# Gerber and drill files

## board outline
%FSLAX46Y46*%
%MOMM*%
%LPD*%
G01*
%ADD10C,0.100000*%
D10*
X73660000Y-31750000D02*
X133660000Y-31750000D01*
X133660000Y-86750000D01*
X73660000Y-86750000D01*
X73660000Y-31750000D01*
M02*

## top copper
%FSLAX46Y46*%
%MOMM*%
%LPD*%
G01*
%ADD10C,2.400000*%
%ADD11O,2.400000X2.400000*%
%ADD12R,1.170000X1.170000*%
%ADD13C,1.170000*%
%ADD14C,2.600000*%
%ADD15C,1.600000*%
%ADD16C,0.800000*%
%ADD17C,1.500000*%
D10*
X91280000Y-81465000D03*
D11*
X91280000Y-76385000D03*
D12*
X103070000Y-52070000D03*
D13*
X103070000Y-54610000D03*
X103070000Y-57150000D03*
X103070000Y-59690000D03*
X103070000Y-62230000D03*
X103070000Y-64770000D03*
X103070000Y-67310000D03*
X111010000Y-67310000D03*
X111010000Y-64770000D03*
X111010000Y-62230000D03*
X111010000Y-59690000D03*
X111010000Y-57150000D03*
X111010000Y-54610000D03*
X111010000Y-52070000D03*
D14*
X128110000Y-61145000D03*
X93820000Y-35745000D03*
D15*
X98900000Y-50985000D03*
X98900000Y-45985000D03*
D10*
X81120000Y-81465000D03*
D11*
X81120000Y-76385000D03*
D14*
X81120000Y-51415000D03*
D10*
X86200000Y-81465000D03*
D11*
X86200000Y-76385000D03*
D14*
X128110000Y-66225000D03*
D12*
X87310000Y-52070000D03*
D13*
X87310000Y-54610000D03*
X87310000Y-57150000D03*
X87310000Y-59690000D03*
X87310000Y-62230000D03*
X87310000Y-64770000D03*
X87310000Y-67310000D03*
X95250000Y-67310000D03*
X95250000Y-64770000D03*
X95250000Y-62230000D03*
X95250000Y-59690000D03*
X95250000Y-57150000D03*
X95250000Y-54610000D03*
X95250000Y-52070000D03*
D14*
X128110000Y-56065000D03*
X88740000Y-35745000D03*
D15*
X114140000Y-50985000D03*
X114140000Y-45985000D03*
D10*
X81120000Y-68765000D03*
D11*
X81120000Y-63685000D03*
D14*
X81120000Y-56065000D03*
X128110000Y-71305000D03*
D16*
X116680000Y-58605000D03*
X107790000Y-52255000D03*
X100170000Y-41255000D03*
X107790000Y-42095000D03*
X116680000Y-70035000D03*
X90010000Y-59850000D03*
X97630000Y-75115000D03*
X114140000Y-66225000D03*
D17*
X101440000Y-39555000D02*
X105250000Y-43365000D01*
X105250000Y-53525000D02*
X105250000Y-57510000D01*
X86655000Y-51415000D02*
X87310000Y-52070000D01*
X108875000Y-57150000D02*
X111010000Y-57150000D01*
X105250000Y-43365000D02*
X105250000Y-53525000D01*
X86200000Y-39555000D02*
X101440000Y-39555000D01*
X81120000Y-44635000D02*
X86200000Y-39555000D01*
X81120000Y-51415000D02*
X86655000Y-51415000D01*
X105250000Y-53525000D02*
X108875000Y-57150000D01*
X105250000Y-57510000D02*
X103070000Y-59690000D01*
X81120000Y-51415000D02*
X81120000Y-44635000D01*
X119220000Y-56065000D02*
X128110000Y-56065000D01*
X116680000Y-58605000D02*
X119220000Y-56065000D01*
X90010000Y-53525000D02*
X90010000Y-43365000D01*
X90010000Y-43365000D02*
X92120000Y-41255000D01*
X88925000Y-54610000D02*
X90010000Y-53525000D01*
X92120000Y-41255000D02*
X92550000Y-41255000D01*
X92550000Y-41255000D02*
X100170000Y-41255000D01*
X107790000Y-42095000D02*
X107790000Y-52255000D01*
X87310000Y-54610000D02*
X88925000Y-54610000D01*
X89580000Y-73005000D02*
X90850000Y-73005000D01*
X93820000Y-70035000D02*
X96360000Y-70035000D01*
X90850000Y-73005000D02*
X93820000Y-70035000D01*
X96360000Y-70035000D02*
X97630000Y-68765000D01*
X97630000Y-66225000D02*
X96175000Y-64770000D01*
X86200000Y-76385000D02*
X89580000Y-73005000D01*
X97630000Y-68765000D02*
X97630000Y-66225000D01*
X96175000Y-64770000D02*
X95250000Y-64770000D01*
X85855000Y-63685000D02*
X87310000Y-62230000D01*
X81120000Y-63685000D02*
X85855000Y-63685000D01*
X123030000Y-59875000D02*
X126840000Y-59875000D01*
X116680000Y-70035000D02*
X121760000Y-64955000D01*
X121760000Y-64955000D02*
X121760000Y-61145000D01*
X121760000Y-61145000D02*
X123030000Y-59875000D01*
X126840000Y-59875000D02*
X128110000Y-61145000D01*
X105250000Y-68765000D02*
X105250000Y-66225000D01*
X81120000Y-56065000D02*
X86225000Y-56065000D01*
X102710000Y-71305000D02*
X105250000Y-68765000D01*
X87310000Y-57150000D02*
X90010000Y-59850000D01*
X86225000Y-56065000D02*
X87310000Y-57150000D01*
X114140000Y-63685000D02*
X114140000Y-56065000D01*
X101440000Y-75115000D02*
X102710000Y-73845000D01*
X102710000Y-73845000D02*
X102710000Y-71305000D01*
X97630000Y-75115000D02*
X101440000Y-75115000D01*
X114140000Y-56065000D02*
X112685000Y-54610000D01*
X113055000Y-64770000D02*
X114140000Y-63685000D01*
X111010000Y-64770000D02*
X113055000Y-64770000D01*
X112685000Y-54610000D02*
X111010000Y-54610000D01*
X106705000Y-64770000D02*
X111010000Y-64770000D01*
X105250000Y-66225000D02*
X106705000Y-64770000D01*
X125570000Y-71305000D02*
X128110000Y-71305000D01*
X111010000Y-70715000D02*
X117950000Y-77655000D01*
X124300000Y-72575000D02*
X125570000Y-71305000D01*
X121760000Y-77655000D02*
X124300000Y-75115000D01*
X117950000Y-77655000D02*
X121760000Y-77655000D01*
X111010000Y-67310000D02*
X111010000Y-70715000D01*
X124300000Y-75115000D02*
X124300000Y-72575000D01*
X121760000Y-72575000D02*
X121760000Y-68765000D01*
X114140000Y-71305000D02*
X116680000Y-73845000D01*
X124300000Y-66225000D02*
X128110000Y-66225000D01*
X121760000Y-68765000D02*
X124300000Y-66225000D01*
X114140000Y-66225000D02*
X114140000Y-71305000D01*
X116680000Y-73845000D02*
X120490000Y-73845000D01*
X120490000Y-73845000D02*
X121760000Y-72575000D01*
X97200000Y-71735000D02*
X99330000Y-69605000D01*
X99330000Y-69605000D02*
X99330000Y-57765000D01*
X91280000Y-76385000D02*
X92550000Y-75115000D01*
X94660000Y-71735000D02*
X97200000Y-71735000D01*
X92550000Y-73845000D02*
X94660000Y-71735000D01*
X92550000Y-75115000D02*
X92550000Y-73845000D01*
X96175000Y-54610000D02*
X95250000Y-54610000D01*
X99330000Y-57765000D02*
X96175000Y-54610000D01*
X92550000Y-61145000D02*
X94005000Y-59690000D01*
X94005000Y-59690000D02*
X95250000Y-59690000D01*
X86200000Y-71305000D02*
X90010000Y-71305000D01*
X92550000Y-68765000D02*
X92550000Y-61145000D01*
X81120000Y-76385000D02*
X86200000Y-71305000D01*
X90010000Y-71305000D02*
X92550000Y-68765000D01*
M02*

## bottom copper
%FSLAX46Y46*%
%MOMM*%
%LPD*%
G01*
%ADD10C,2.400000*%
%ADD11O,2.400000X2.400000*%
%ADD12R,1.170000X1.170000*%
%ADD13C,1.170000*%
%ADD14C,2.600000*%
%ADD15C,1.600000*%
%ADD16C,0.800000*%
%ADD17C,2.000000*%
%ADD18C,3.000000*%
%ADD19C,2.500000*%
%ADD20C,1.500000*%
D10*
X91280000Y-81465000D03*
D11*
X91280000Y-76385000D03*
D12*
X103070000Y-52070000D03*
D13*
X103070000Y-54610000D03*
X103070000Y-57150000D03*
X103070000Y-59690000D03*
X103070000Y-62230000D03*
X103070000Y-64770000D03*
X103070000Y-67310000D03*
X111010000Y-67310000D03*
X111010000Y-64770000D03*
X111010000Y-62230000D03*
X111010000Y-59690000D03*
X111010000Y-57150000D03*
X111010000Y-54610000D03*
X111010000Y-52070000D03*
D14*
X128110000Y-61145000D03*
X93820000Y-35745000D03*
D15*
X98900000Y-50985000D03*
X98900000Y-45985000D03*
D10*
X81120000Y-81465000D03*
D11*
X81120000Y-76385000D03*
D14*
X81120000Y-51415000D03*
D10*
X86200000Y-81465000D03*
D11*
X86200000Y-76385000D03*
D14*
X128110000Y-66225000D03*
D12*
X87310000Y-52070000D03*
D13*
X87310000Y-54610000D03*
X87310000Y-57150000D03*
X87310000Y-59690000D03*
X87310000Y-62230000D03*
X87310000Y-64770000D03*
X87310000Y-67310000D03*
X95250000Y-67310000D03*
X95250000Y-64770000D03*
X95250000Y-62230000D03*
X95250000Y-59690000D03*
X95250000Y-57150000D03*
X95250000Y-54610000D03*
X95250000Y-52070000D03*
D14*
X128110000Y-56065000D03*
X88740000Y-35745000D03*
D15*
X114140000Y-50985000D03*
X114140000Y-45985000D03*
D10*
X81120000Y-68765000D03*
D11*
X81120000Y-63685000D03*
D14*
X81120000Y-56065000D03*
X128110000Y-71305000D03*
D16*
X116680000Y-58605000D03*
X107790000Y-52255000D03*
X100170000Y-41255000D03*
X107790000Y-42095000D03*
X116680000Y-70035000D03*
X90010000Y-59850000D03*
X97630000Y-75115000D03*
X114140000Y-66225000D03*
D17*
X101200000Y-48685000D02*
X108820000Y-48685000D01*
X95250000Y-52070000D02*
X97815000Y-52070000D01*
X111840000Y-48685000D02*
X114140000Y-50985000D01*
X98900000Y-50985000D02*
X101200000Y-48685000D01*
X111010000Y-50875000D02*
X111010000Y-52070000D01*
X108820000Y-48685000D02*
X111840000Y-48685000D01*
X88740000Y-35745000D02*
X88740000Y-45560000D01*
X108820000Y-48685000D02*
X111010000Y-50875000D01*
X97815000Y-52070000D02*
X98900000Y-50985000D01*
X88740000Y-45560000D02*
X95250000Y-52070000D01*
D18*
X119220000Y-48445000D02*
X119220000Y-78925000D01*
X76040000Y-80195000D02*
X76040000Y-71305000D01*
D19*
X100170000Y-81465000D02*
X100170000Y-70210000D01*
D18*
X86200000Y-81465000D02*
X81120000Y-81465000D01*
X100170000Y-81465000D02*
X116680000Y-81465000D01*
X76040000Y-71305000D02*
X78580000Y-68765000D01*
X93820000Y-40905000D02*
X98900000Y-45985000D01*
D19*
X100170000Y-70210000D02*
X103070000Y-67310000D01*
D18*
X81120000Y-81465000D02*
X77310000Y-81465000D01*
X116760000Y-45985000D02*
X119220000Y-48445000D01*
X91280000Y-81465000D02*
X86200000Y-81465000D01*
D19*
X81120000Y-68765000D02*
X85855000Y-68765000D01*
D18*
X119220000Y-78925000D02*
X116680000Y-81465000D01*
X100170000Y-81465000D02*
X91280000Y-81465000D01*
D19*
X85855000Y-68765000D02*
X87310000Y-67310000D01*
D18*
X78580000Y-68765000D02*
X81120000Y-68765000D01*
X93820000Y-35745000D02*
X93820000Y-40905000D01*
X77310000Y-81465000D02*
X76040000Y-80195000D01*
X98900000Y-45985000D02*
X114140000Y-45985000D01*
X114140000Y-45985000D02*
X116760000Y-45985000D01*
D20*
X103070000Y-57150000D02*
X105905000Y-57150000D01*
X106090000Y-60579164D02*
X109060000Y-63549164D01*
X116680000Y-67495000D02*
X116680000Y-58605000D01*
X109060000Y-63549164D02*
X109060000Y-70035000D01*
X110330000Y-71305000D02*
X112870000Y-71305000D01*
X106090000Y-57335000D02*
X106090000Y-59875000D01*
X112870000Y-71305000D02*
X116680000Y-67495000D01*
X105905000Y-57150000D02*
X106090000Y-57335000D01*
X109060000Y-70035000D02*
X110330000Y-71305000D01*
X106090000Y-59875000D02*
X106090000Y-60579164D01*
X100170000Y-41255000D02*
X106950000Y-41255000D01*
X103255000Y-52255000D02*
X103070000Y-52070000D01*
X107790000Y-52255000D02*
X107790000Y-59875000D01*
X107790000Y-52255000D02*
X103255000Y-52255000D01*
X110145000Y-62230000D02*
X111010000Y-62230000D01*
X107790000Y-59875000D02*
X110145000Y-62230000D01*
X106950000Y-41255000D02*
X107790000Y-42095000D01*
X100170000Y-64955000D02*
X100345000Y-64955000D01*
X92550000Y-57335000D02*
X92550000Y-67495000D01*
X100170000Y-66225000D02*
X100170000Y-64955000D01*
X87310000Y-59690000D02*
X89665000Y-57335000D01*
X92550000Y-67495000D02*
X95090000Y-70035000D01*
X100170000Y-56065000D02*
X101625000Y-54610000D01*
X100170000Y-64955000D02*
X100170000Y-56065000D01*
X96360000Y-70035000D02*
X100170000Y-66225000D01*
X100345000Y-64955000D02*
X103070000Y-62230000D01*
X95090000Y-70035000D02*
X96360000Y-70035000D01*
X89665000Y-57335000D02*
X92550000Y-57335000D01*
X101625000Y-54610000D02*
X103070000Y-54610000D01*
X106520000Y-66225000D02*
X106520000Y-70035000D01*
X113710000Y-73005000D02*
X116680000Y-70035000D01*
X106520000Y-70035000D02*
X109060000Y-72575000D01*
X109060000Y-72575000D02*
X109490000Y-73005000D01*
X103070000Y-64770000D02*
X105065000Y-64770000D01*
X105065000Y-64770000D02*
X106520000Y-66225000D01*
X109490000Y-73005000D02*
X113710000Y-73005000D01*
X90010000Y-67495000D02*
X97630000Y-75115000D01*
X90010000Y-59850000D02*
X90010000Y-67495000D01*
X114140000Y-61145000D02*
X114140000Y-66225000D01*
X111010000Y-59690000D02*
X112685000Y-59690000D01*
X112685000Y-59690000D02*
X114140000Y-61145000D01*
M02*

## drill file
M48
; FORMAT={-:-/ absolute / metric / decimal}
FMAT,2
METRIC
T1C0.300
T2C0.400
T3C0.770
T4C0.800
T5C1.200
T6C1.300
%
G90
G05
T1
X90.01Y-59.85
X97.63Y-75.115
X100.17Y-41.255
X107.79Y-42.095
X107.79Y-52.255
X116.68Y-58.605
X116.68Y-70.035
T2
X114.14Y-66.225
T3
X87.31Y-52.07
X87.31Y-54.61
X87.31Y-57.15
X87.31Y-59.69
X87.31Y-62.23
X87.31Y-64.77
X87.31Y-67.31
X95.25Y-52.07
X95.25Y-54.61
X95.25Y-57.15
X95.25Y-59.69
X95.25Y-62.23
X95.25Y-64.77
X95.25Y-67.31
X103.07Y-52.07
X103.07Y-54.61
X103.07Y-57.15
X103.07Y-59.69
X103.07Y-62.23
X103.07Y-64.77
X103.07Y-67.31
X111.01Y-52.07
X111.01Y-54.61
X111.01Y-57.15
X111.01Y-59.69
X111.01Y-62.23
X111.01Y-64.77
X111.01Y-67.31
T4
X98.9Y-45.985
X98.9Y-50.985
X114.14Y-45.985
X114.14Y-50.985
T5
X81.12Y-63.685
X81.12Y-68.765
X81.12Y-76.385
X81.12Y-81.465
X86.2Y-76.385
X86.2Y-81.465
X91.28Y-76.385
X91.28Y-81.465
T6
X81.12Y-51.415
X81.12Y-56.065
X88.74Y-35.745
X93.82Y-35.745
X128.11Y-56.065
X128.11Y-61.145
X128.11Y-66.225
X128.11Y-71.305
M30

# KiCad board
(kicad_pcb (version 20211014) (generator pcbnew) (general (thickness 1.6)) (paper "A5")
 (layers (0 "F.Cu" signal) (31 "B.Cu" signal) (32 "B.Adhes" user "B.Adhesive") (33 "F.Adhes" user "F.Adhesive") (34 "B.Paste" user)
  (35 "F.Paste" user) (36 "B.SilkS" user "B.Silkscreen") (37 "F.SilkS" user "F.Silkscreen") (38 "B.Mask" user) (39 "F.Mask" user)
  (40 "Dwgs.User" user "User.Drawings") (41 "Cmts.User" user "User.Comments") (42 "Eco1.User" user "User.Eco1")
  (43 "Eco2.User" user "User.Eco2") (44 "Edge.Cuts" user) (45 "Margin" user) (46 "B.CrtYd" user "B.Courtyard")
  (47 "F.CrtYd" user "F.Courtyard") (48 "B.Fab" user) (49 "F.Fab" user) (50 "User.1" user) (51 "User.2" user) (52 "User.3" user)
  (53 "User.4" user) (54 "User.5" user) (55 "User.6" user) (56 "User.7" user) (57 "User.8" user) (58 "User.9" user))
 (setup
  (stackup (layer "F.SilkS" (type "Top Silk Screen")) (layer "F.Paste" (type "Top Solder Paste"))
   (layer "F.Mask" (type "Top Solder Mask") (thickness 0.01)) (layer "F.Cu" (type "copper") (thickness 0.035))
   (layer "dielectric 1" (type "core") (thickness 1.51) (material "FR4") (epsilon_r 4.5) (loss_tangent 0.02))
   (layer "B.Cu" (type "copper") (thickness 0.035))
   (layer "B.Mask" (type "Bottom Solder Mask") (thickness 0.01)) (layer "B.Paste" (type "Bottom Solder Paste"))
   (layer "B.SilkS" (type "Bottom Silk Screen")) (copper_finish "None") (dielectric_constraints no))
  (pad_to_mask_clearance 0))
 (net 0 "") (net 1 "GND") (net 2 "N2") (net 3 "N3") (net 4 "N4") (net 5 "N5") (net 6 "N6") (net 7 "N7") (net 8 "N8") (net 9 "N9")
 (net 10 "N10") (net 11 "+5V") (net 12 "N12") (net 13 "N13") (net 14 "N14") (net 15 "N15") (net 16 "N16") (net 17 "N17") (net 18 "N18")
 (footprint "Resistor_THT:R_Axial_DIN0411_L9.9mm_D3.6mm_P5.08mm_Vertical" (layer "F.Cu") (at 91.28 81.465 90)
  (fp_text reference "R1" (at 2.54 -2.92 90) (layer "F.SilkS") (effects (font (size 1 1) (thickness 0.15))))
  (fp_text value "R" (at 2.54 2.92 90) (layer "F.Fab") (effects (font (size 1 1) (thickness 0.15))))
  (pad "1" thru_hole circle (at 0 0 90) (size 2.4 2.4) (drill 1.2) (layers *.Cu *.Mask) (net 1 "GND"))
  (pad "2" thru_hole oval (at 5.08 0 90) (size 2.4 2.4) (drill 1.2) (layers *.Cu *.Mask) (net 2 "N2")))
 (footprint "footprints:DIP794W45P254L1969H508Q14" (layer "F.Cu") (at 107.04 59.69)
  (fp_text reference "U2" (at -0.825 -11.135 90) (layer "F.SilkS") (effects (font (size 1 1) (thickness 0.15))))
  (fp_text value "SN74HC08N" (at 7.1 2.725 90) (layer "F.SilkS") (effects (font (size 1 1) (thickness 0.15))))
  (pad "1" thru_hole rect locked (at -3.97 -7.62) (size 1.17 1.17) (drill 0.77) (layers *.Cu *.Mask) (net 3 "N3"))
  (pad "2" thru_hole circle locked (at -3.97 -5.08) (size 1.17 1.17) (drill 0.77) (layers *.Cu *.Mask) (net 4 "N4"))
  (pad "3" thru_hole circle locked (at -3.97 -2.54) (size 1.17 1.17) (drill 0.77) (layers *.Cu *.Mask) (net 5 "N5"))
  (pad "4" thru_hole circle locked (at -3.97 0) (size 1.17 1.17) (drill 0.77) (layers *.Cu *.Mask) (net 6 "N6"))
  (pad "5" thru_hole circle locked (at -3.97 2.54) (size 1.17 1.17) (drill 0.77) (layers *.Cu *.Mask) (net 4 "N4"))
  (pad "6" thru_hole circle locked (at -3.97 5.08) (size 1.17 1.17) (drill 0.77) (layers *.Cu *.Mask) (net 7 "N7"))
  (pad "7" thru_hole circle locked (at -3.97 7.62) (size 1.17 1.17) (drill 0.77) (layers *.Cu *.Mask) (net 1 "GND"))
  (pad "8" thru_hole circle locked (at 3.97 7.62) (size 1.17 1.17) (drill 0.77) (layers *.Cu *.Mask) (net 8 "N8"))
  (pad "9" thru_hole circle locked (at 3.97 5.08) (size 1.17 1.17) (drill 0.77) (layers *.Cu *.Mask) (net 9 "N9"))
  (pad "10" thru_hole circle locked (at 3.97 2.54) (size 1.17 1.17) (drill 0.77) (layers *.Cu *.Mask) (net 3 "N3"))
  (pad "11" thru_hole circle locked (at 3.97 0) (size 1.17 1.17) (drill 0.77) (layers *.Cu *.Mask) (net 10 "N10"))
  (pad "12" thru_hole circle locked (at 3.97 -2.54) (size 1.17 1.17) (drill 0.77) (layers *.Cu *.Mask) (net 6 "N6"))
  (pad "13" thru_hole circle locked (at 3.97 -5.08) (size 1.17 1.17) (drill 0.77) (layers *.Cu *.Mask) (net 9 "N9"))
  (pad "14" thru_hole circle locked (at 3.97 -7.62) (size 1.17 1.17) (drill 0.77) (layers *.Cu *.Mask) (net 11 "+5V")))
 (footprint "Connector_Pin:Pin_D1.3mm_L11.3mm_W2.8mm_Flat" (layer "F.Cu") (at 128.11 61.145)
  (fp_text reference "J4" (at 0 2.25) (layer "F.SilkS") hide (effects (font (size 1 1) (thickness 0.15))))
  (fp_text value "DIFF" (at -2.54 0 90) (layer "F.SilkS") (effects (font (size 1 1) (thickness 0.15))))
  (pad "1" thru_hole circle (at 0 0) (size 2.6 2.6) (drill 1.3) (layers *.Cu *.Mask) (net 7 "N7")))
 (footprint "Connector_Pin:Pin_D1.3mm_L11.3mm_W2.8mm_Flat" (layer "F.Cu") (at 93.82 35.745)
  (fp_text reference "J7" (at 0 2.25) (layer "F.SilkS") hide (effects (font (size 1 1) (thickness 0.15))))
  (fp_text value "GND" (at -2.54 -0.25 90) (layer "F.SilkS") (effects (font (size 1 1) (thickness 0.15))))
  (pad "1" thru_hole circle (at 0 0) (size 2.6 2.6) (drill 1.3) (layers *.Cu *.Mask) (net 1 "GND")))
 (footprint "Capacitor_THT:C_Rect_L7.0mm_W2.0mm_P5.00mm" (layer "F.Cu") (at 98.9 50.985 90)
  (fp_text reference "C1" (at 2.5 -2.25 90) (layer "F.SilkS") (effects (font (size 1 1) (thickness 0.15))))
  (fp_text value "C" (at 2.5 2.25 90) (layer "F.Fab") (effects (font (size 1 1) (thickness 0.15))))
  (pad "1" thru_hole circle (at 0 0 90) (size 1.6 1.6) (drill 0.8) (layers *.Cu *.Mask) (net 11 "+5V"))
  (pad "2" thru_hole circle (at 5 0 90) (size 1.6 1.6) (drill 0.8) (layers *.Cu *.Mask) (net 1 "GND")))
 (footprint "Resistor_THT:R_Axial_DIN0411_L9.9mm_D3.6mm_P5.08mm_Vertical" (layer "F.Cu") (at 81.12 81.465 90)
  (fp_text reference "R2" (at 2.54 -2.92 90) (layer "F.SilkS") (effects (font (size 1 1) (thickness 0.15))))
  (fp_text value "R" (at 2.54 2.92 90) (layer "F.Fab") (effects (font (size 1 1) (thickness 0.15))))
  (pad "1" thru_hole circle (at 0 0 90) (size 2.4 2.4) (drill 1.2) (layers *.Cu *.Mask) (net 1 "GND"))
  (pad "2" thru_hole oval (at 5.08 0 90) (size 2.4 2.4) (drill 1.2) (layers *.Cu *.Mask) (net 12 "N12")))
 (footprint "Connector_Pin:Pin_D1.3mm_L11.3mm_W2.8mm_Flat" (layer "F.Cu") (at 81.12 51.415 180)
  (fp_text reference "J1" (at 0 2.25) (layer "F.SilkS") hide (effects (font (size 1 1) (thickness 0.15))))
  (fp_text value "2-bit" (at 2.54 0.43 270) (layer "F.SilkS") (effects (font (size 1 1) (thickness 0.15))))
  (pad "1" thru_hole circle (at 0 0 180) (size 2.6 2.6) (drill 1.3) (layers *.Cu *.Mask) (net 6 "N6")))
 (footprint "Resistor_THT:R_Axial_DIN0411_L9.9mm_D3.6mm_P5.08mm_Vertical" (layer "F.Cu") (at 86.2 81.465 90)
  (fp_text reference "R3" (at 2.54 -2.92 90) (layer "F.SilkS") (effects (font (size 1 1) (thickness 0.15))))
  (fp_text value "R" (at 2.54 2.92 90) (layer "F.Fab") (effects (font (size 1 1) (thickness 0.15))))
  (pad "1" thru_hole circle (at 0 0 90) (size 2.4 2.4) (drill 1.2) (layers *.Cu *.Mask) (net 1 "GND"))
  (pad "2" thru_hole oval (at 5.08 0 90) (size 2.4 2.4) (drill 1.2) (layers *.Cu *.Mask) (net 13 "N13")))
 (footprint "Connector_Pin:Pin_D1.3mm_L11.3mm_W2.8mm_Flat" (layer "F.Cu") (at 128.11 66.225)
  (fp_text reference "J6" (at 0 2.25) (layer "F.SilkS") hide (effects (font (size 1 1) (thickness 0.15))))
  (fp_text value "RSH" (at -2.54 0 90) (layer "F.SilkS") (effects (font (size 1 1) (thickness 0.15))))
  (pad "1" thru_hole circle (at 0 0) (size 2.6 2.6) (drill 1.3) (layers *.Cu *.Mask) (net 10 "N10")))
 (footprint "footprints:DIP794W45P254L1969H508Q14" (layer "F.Cu") (at 91.28 59.69)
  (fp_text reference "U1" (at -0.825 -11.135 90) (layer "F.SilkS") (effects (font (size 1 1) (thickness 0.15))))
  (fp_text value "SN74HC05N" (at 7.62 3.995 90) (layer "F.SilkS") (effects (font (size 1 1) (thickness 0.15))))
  (pad "1" thru_hole rect locked (at -3.97 -7.62) (size 1.17 1.17) (drill 0.77) (layers *.Cu *.Mask) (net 6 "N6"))
  (pad "2" thru_hole circle locked (at -3.97 -5.08) (size 1.17 1.17) (drill 0.77) (layers *.Cu *.Mask) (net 3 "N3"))
  (pad "3" thru_hole circle locked (at -3.97 -2.54) (size 1.17 1.17) (drill 0.77) (layers *.Cu *.Mask) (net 9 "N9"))
  (pad "4" thru_hole circle locked (at -3.97 0) (size 1.17 1.17) (drill 0.77) (layers *.Cu *.Mask) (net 4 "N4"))
  (pad "5" thru_hole circle locked (at -3.97 2.54) (size 1.17 1.17) (drill 0.77) (layers *.Cu *.Mask) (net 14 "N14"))
  (pad "6" thru_hole circle locked (at -3.97 5.08) (size 1.17 1.17) (drill 0.77) (layers *.Cu *.Mask) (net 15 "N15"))
  (pad "7" thru_hole circle locked (at -3.97 7.62) (size 1.17 1.17) (drill 0.77) (layers *.Cu *.Mask) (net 1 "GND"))
  (pad "8" thru_hole circle locked (at 3.97 7.62) (size 1.17 1.17) (drill 0.77) (layers *.Cu *.Mask) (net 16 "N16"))
  (pad "9" thru_hole circle locked (at 3.97 5.08) (size 1.17 1.17) (drill 0.77) (layers *.Cu *.Mask) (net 13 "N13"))
  (pad "10" thru_hole circle locked (at 3.97 2.54) (size 1.17 1.17) (drill 0.77) (layers *.Cu *.Mask) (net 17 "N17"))
  (pad "11" thru_hole circle locked (at 3.97 0) (size 1.17 1.17) (drill 0.77) (layers *.Cu *.Mask) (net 12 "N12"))
  (pad "12" thru_hole circle locked (at 3.97 -2.54) (size 1.17 1.17) (drill 0.77) (layers *.Cu *.Mask) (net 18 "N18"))
  (pad "13" thru_hole circle locked (at 3.97 -5.08) (size 1.17 1.17) (drill 0.77) (layers *.Cu *.Mask) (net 2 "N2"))
  (pad "14" thru_hole circle locked (at 3.97 -7.62) (size 1.17 1.17) (drill 0.77) (layers *.Cu *.Mask) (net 11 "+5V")))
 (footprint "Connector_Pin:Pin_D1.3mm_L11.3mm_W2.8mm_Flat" (layer "F.Cu") (at 128.11 56.065)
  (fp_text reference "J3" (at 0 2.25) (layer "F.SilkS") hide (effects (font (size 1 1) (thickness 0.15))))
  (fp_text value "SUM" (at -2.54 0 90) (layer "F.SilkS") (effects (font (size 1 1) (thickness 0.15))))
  (pad "1" thru_hole circle (at 0 0) (size 2.6 2.6) (drill 1.3) (layers *.Cu *.Mask) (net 5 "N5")))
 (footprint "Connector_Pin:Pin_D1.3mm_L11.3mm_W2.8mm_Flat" (layer "F.Cu") (at 88.74 35.745)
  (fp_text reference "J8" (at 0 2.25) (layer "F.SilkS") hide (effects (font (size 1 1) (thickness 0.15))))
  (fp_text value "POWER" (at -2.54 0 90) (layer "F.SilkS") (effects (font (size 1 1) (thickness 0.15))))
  (pad "1" thru_hole circle (at 0 0) (size 2.6 2.6) (drill 1.3) (layers *.Cu *.Mask) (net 11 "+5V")))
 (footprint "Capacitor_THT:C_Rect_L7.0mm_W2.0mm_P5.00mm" (layer "F.Cu") (at 114.14 50.985 90)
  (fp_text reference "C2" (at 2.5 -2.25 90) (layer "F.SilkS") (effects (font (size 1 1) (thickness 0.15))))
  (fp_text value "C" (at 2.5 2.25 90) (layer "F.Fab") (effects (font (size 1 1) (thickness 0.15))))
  (pad "1" thru_hole circle (at 0 0 90) (size 1.6 1.6) (drill 0.8) (layers *.Cu *.Mask) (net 11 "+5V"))
  (pad "2" thru_hole circle (at 5 0 90) (size 1.6 1.6) (drill 0.8) (layers *.Cu *.Mask) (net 1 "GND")))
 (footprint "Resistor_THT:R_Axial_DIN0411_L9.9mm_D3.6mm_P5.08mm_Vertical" (layer "F.Cu") (at 81.12 68.765 90)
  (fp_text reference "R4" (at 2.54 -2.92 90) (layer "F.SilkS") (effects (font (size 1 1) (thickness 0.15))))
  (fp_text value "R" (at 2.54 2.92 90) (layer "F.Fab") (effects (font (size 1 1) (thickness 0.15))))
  (pad "1" thru_hole circle (at 0 0 90) (size 2.4 2.4) (drill 1.2) (layers *.Cu *.Mask) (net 1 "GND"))
  (pad "2" thru_hole oval (at 5.08 0 90) (size 2.4 2.4) (drill 1.2) (layers *.Cu *.Mask) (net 14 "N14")))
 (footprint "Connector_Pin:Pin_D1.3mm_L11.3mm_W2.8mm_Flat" (layer "F.Cu") (at 81.12 56.065)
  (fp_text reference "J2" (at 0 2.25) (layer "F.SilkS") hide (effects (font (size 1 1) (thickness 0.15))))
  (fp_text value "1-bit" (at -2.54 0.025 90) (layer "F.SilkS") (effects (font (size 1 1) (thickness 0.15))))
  (pad "1" thru_hole circle (at 0 0) (size 2.6 2.6) (drill 1.3) (layers *.Cu *.Mask) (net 9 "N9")))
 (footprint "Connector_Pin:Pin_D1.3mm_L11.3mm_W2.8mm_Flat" (layer "F.Cu") (at 128.11 71.305)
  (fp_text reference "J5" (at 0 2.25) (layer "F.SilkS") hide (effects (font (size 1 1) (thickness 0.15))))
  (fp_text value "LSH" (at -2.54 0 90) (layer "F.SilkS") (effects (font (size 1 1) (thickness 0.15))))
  (pad "1" thru_hole circle (at 0 0) (size 2.6 2.6) (drill 1.3) (layers *.Cu *.Mask) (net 8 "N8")))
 (gr_rect (start 73.66 31.75) (end 133.66 86.75) (layer "Edge.Cuts") (width 0.1) (fill none))
 (segment (start 101.2 48.685) (end 108.82 48.685) (width 2) (layer "B.Cu") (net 11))
 (segment (start 95.25 52.07) (end 97.815 52.07) (width 2) (layer "B.Cu") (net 11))
 (segment (start 111.84 48.685) (end 114.14 50.985) (width 2) (layer "B.Cu") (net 11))
 (segment (start 98.9 50.985) (end 101.2 48.685) (width 2) (layer "B.Cu") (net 11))
 (segment (start 111.01 50.875) (end 111.01 52.07) (width 2) (layer "B.Cu") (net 11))
 (segment (start 108.82 48.685) (end 111.84 48.685) (width 2) (layer "B.Cu") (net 11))
 (segment (start 88.74 35.745) (end 88.74 45.56) (width 2) (layer "B.Cu") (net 11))
 (segment (start 108.82 48.685) (end 111.01 50.875) (width 2) (layer "B.Cu") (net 11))
 (segment (start 97.815 52.07) (end 98.9 50.985) (width 2) (layer "B.Cu") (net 11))
 (segment (start 88.74 45.56) (end 95.25 52.07) (width 2) (layer "B.Cu") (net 11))
 (segment (start 119.22 48.445) (end 119.22 78.925) (width 3) (layer "B.Cu") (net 1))
 (segment (start 76.04 80.195) (end 76.04 71.305) (width 3) (layer "B.Cu") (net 1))
 (segment (start 100.17 81.465) (end 100.17 70.21) (width 2.5) (layer "B.Cu") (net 1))
 (segment (start 86.2 81.465) (end 81.12 81.465) (width 3) (layer "B.Cu") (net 1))
 (segment (start 100.17 81.465) (end 116.68 81.465) (width 3) (layer "B.Cu") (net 1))
 (segment (start 76.04 71.305) (end 78.58 68.765) (width 3) (layer "B.Cu") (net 1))
 (segment (start 93.82 40.905) (end 98.9 45.985) (width 3) (layer "B.Cu") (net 1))
 (segment (start 100.17 70.21) (end 103.07 67.31) (width 2.5) (layer "B.Cu") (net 1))
 (segment (start 81.12 81.465) (end 77.31 81.465) (width 3) (layer "B.Cu") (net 1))
 (segment (start 116.76 45.985) (end 119.22 48.445) (width 3) (layer "B.Cu") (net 1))
 (segment (start 91.28 81.465) (end 86.2 81.465) (width 3) (layer "B.Cu") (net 1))
 (segment (start 81.12 68.765) (end 85.855 68.765) (width 2.5) (layer "B.Cu") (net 1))
 (segment (start 119.22 78.925) (end 116.68 81.465) (width 3) (layer "B.Cu") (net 1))
 (segment (start 100.17 81.465) (end 91.28 81.465) (width 3) (layer "B.Cu") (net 1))
 (segment (start 85.855 68.765) (end 87.31 67.31) (width 2.5) (layer "B.Cu") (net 1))
 (segment (start 78.58 68.765) (end 81.12 68.765) (width 3) (layer "B.Cu") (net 1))
 (segment (start 93.82 35.745) (end 93.82 40.905) (width 3) (layer "B.Cu") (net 1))
 (segment (start 77.31 81.465) (end 76.04 80.195) (width 3) (layer "B.Cu") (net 1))
 (segment (start 98.9 45.985) (end 114.14 45.985) (width 3) (layer "B.Cu") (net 1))
 (segment (start 114.14 45.985) (end 116.76 45.985) (width 3) (layer "B.Cu") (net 1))
 (segment (start 101.44 39.555) (end 105.25 43.365) (width 1.5) (layer "F.Cu") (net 6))
 (segment (start 105.25 53.525) (end 105.25 57.51) (width 1.5) (layer "F.Cu") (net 6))
 (segment (start 86.655 51.415) (end 87.31 52.07) (width 1.5) (layer "F.Cu") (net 6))
 (segment (start 108.875 57.15) (end 111.01 57.15) (width 1.5) (layer "F.Cu") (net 6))
 (segment (start 105.25 43.365) (end 105.25 53.525) (width 1.5) (layer "F.Cu") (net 6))
 (segment (start 86.2 39.555) (end 101.44 39.555) (width 1.5) (layer "F.Cu") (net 6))
 (segment (start 81.12 44.635) (end 86.2 39.555) (width 1.5) (layer "F.Cu") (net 6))
 (segment (start 81.12 51.415) (end 86.655 51.415) (width 1.5) (layer "F.Cu") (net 6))
 (segment (start 105.25 53.525) (end 108.875 57.15) (width 1.5) (layer "F.Cu") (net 6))
 (segment (start 105.25 57.51) (end 103.07 59.69) (width 1.5) (layer "F.Cu") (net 6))
 (segment (start 81.12 51.415) (end 81.12 44.635) (width 1.5) (layer "F.Cu") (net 6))
 (segment (start 119.22 56.065) (end 128.11 56.065) (width 1.5) (layer "F.Cu") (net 5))
 (segment (start 116.68 58.605) (end 119.22 56.065) (width 1.5) (layer "F.Cu") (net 5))
 (via (at 116.68 58.605) (size 0.8) (drill 0.3) (layers "F.Cu" "B.Cu") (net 5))
 (segment (start 103.07 57.15) (end 105.905 57.15) (width 1.5) (layer "B.Cu") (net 5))
 (segment (start 106.09 60.579164) (end 109.06 63.549164) (width 1.5) (layer "B.Cu") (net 5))
 (segment (start 116.68 67.495) (end 116.68 58.605) (width 1.5) (layer "B.Cu") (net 5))
 (segment (start 109.06 63.549164) (end 109.06 70.035) (width 1.5) (layer "B.Cu") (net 5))
 (segment (start 110.33 71.305) (end 112.87 71.305) (width 1.5) (layer "B.Cu") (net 5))
 (segment (start 106.09 57.335) (end 106.09 59.875) (width 1.5) (layer "B.Cu") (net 5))
 (segment (start 112.87 71.305) (end 116.68 67.495) (width 1.5) (layer "B.Cu") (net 5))
 (segment (start 105.905 57.15) (end 106.09 57.335) (width 1.5) (layer "B.Cu") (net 5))
 (segment (start 109.06 70.035) (end 110.33 71.305) (width 1.5) (layer "B.Cu") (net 5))
 (segment (start 106.09 59.875) (end 106.09 60.579164) (width 1.5) (layer "B.Cu") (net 5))
 (segment (start 90.01 53.525) (end 90.01 43.365) (width 1.5) (layer "F.Cu") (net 3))
 (segment (start 90.01 43.365) (end 92.12 41.255) (width 1.5) (layer "F.Cu") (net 3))
 (segment (start 88.925 54.61) (end 90.01 53.525) (width 1.5) (layer "F.Cu") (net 3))
 (segment (start 92.12 41.255) (end 92.55 41.255) (width 1.5) (layer "F.Cu") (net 3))
 (segment (start 92.55 41.255) (end 100.17 41.255) (width 1.5) (layer "F.Cu") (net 3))
 (segment (start 107.79 42.095) (end 107.79 52.255) (width 1.5) (layer "F.Cu") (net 3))
 (segment (start 87.31 54.61) (end 88.925 54.61) (width 1.5) (layer "F.Cu") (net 3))
 (via (at 107.79 52.255) (size 0.8) (drill 0.3) (layers "F.Cu" "B.Cu") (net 3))
 (via (at 100.17 41.255) (size 0.8) (drill 0.3) (layers "F.Cu" "B.Cu") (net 3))
 (via (at 107.79 42.095) (size 0.8) (drill 0.3) (layers "F.Cu" "B.Cu") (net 3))
 (segment (start 100.17 41.255) (end 106.95 41.255) (width 1.5) (layer "B.Cu") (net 3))
 (segment (start 103.255 52.255) (end 103.07 52.07) (width 1.5) (layer "B.Cu") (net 3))
 (segment (start 107.79 52.255) (end 107.79 59.875) (width 1.5) (layer "B.Cu") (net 3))
 (segment (start 107.79 52.255) (end 103.255 52.255) (width 1.5) (layer "B.Cu") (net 3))
 (segment (start 110.145 62.23) (end 111.01 62.23) (width 1.5) (layer "B.Cu") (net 3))
 (segment (start 107.79 59.875) (end 110.145 62.23) (width 1.5) (layer "B.Cu") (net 3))
 (segment (start 106.95 41.255) (end 107.79 42.095) (width 1.5) (layer "B.Cu") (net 3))
 (segment (start 100.17 64.955) (end 100.345 64.955) (width 1.5) (layer "B.Cu") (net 4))
 (segment (start 92.55 57.335) (end 92.55 67.495) (width 1.5) (layer "B.Cu") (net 4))
 (segment (start 100.17 66.225) (end 100.17 64.955) (width 1.5) (layer "B.Cu") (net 4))
 (segment (start 87.31 59.69) (end 89.665 57.335) (width 1.5) (layer "B.Cu") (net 4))
 (segment (start 92.55 67.495) (end 95.09 70.035) (width 1.5) (layer "B.Cu") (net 4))
 (segment (start 100.17 56.065) (end 101.625 54.61) (width 1.5) (layer "B.Cu") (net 4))
 (segment (start 100.17 64.955) (end 100.17 56.065) (width 1.5) (layer "B.Cu") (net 4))
 (segment (start 96.36 70.035) (end 100.17 66.225) (width 1.5) (layer "B.Cu") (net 4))
 (segment (start 100.345 64.955) (end 103.07 62.23) (width 1.5) (layer "B.Cu") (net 4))
 (segment (start 95.09 70.035) (end 96.36 70.035) (width 1.5) (layer "B.Cu") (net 4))
 (segment (start 89.665 57.335) (end 92.55 57.335) (width 1.5) (layer "B.Cu") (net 4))
 (segment (start 101.625 54.61) (end 103.07 54.61) (width 1.5) (layer "B.Cu") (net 4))
 (segment (start 89.58 73.005) (end 90.85 73.005) (width 1.5) (layer "F.Cu") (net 13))
 (segment (start 93.82 70.035) (end 96.36 70.035) (width 1.5) (layer "F.Cu") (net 13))
 (segment (start 90.85 73.005) (end 93.82 70.035) (width 1.5) (layer "F.Cu") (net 13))
 (segment (start 96.36 70.035) (end 97.63 68.765) (width 1.5) (layer "F.Cu") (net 13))
 (segment (start 97.63 66.225) (end 96.175 64.77) (width 1.5) (layer "F.Cu") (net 13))
 (segment (start 86.2 76.385) (end 89.58 73.005) (width 1.5) (layer "F.Cu") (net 13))
 (segment (start 97.63 68.765) (end 97.63 66.225) (width 1.5) (layer "F.Cu") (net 13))
 (segment (start 96.175 64.77) (end 95.25 64.77) (width 1.5) (layer "F.Cu") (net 13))
 (segment (start 85.855 63.685) (end 87.31 62.23) (width 1.5) (layer "F.Cu") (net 14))
 (segment (start 81.12 63.685) (end 85.855 63.685) (width 1.5) (layer "F.Cu") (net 14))
 (segment (start 123.03 59.875) (end 126.84 59.875) (width 1.5) (layer "F.Cu") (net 7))
 (segment (start 116.68 70.035) (end 121.76 64.955) (width 1.5) (layer "F.Cu") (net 7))
 (segment (start 121.76 64.955) (end 121.76 61.145) (width 1.5) (layer "F.Cu") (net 7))
 (segment (start 121.76 61.145) (end 123.03 59.875) (width 1.5) (layer "F.Cu") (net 7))
 (segment (start 126.84 59.875) (end 128.11 61.145) (width 1.5) (layer "F.Cu") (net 7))
 (via (at 116.68 70.035) (size 0.8) (drill 0.3) (layers "F.Cu" "B.Cu") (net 7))
 (segment (start 106.52 66.225) (end 106.52 70.035) (width 1.5) (layer "B.Cu") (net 7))
 (segment (start 113.71 73.005) (end 116.68 70.035) (width 1.5) (layer "B.Cu") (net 7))
 (segment (start 106.52 70.035) (end 109.06 72.575) (width 1.5) (layer "B.Cu") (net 7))
 (segment (start 109.06 72.575) (end 109.49 73.005) (width 1.5) (layer "B.Cu") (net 7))
 (segment (start 103.07 64.77) (end 105.065 64.77) (width 1.5) (layer "B.Cu") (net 7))
 (segment (start 105.065 64.77) (end 106.52 66.225) (width 1.5) (layer "B.Cu") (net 7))
 (segment (start 109.49 73.005) (end 113.71 73.005) (width 1.5) (layer "B.Cu") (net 7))
 (segment (start 105.25 68.765) (end 105.25 66.225) (width 1.5) (layer "F.Cu") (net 9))
 (segment (start 81.12 56.065) (end 86.225 56.065) (width 1.5) (layer "F.Cu") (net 9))
 (segment (start 102.71 71.305) (end 105.25 68.765) (width 1.5) (layer "F.Cu") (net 9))
 (segment (start 87.31 57.15) (end 90.01 59.85) (width 1.5) (layer "F.Cu") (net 9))
 (segment (start 86.225 56.065) (end 87.31 57.15) (width 1.5) (layer "F.Cu") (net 9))
 (segment (start 114.14 63.685) (end 114.14 56.065) (width 1.5) (layer "F.Cu") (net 9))
 (segment (start 101.44 75.115) (end 102.71 73.845) (width 1.5) (layer "F.Cu") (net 9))
 (segment (start 102.71 73.845) (end 102.71 71.305) (width 1.5) (layer "F.Cu") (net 9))
 (segment (start 97.63 75.115) (end 101.44 75.115) (width 1.5) (layer "F.Cu") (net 9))
 (segment (start 114.14 56.065) (end 112.685 54.61) (width 1.5) (layer "F.Cu") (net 9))
 (segment (start 113.055 64.77) (end 114.14 63.685) (width 1.5) (layer "F.Cu") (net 9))
 (segment (start 111.01 64.77) (end 113.055 64.77) (width 1.5) (layer "F.Cu") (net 9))
 (segment (start 112.685 54.61) (end 111.01 54.61) (width 1.5) (layer "F.Cu") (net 9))
 (segment (start 106.705 64.77) (end 111.01 64.77) (width 1.5) (layer "F.Cu") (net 9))
 (segment (start 105.25 66.225) (end 106.705 64.77) (width 1.5) (layer "F.Cu") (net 9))
 (via (at 90.01 59.85) (size 0.8) (drill 0.3) (layers "F.Cu" "B.Cu") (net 9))
 (via (at 97.63 75.115) (size 0.8) (drill 0.3) (layers "F.Cu" "B.Cu") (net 9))
 (segment (start 90.01 67.495) (end 97.63 75.115) (width 1.5) (layer "B.Cu") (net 9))
 (segment (start 90.01 59.85) (end 90.01 67.495) (width 1.5) (layer "B.Cu") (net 9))
 (segment (start 125.57 71.305) (end 128.11 71.305) (width 1.5) (layer "F.Cu") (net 8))
 (segment (start 111.01 70.715) (end 117.95 77.655) (width 1.5) (layer "F.Cu") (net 8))
 (segment (start 124.3 72.575) (end 125.57 71.305) (width 1.5) (layer "F.Cu") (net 8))
 (segment (start 121.76 77.655) (end 124.3 75.115) (width 1.5) (layer "F.Cu") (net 8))
 (segment (start 117.95 77.655) (end 121.76 77.655) (width 1.5) (layer "F.Cu") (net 8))
 (segment (start 111.01 67.31) (end 111.01 70.715) (width 1.5) (layer "F.Cu") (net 8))
 (segment (start 124.3 75.115) (end 124.3 72.575) (width 1.5) (layer "F.Cu") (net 8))
 (segment (start 121.76 72.575) (end 121.76 68.765) (width 1.5) (layer "F.Cu") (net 10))
 (segment (start 114.14 71.305) (end 116.68 73.845) (width 1.5) (layer "F.Cu") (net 10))
 (segment (start 124.3 66.225) (end 128.11 66.225) (width 1.5) (layer "F.Cu") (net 10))
 (segment (start 121.76 68.765) (end 124.3 66.225) (width 1.5) (layer "F.Cu") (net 10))
 (segment (start 114.14 66.225) (end 114.14 71.305) (width 1.5) (layer "F.Cu") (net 10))
 (segment (start 116.68 73.845) (end 120.49 73.845) (width 1.5) (layer "F.Cu") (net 10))
 (segment (start 120.49 73.845) (end 121.76 72.575) (width 1.5) (layer "F.Cu") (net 10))
 (via (at 114.14 66.225) (size 0.8) (drill 0.4) (layers "F.Cu" "B.Cu") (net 10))
 (segment (start 114.14 61.145) (end 114.14 66.225) (width 1.5) (layer "B.Cu") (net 10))
 (segment (start 111.01 59.69) (end 112.685 59.69) (width 1.5) (layer "B.Cu") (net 10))
 (segment (start 112.685 59.69) (end 114.14 61.145) (width 1.5) (layer "B.Cu") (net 10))
 (segment (start 97.2 71.735) (end 99.33 69.605) (width 1.5) (layer "F.Cu") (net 2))
 (segment (start 99.33 69.605) (end 99.33 57.765) (width 1.5) (layer "F.Cu") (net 2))
 (segment (start 91.28 76.385) (end 92.55 75.115) (width 1.5) (layer "F.Cu") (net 2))
 (segment (start 94.66 71.735) (end 97.2 71.735) (width 1.5) (layer "F.Cu") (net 2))
 (segment (start 92.55 73.845) (end 94.66 71.735) (width 1.5) (layer "F.Cu") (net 2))
 (segment (start 92.55 75.115) (end 92.55 73.845) (width 1.5) (layer "F.Cu") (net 2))
 (segment (start 96.175 54.61) (end 95.25 54.61) (width 1.5) (layer "F.Cu") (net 2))
 (segment (start 99.33 57.765) (end 96.175 54.61) (width 1.5) (layer "F.Cu") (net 2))
 (segment (start 92.55 61.145) (end 94.005 59.69) (width 1.5) (layer "F.Cu") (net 12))
 (segment (start 94.005 59.69) (end 95.25 59.69) (width 1.5) (layer "F.Cu") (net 12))
 (segment (start 86.2 71.305) (end 90.01 71.305) (width 1.5) (layer "F.Cu") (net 12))
 (segment (start 92.55 68.765) (end 92.55 61.145) (width 1.5) (layer "F.Cu") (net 12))
 (segment (start 81.12 76.385) (end 86.2 71.305) (width 1.5) (layer "F.Cu") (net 12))
 (segment (start 90.01 71.305) (end 92.55 68.765) (width 1.5) (layer "F.Cu") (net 12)))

